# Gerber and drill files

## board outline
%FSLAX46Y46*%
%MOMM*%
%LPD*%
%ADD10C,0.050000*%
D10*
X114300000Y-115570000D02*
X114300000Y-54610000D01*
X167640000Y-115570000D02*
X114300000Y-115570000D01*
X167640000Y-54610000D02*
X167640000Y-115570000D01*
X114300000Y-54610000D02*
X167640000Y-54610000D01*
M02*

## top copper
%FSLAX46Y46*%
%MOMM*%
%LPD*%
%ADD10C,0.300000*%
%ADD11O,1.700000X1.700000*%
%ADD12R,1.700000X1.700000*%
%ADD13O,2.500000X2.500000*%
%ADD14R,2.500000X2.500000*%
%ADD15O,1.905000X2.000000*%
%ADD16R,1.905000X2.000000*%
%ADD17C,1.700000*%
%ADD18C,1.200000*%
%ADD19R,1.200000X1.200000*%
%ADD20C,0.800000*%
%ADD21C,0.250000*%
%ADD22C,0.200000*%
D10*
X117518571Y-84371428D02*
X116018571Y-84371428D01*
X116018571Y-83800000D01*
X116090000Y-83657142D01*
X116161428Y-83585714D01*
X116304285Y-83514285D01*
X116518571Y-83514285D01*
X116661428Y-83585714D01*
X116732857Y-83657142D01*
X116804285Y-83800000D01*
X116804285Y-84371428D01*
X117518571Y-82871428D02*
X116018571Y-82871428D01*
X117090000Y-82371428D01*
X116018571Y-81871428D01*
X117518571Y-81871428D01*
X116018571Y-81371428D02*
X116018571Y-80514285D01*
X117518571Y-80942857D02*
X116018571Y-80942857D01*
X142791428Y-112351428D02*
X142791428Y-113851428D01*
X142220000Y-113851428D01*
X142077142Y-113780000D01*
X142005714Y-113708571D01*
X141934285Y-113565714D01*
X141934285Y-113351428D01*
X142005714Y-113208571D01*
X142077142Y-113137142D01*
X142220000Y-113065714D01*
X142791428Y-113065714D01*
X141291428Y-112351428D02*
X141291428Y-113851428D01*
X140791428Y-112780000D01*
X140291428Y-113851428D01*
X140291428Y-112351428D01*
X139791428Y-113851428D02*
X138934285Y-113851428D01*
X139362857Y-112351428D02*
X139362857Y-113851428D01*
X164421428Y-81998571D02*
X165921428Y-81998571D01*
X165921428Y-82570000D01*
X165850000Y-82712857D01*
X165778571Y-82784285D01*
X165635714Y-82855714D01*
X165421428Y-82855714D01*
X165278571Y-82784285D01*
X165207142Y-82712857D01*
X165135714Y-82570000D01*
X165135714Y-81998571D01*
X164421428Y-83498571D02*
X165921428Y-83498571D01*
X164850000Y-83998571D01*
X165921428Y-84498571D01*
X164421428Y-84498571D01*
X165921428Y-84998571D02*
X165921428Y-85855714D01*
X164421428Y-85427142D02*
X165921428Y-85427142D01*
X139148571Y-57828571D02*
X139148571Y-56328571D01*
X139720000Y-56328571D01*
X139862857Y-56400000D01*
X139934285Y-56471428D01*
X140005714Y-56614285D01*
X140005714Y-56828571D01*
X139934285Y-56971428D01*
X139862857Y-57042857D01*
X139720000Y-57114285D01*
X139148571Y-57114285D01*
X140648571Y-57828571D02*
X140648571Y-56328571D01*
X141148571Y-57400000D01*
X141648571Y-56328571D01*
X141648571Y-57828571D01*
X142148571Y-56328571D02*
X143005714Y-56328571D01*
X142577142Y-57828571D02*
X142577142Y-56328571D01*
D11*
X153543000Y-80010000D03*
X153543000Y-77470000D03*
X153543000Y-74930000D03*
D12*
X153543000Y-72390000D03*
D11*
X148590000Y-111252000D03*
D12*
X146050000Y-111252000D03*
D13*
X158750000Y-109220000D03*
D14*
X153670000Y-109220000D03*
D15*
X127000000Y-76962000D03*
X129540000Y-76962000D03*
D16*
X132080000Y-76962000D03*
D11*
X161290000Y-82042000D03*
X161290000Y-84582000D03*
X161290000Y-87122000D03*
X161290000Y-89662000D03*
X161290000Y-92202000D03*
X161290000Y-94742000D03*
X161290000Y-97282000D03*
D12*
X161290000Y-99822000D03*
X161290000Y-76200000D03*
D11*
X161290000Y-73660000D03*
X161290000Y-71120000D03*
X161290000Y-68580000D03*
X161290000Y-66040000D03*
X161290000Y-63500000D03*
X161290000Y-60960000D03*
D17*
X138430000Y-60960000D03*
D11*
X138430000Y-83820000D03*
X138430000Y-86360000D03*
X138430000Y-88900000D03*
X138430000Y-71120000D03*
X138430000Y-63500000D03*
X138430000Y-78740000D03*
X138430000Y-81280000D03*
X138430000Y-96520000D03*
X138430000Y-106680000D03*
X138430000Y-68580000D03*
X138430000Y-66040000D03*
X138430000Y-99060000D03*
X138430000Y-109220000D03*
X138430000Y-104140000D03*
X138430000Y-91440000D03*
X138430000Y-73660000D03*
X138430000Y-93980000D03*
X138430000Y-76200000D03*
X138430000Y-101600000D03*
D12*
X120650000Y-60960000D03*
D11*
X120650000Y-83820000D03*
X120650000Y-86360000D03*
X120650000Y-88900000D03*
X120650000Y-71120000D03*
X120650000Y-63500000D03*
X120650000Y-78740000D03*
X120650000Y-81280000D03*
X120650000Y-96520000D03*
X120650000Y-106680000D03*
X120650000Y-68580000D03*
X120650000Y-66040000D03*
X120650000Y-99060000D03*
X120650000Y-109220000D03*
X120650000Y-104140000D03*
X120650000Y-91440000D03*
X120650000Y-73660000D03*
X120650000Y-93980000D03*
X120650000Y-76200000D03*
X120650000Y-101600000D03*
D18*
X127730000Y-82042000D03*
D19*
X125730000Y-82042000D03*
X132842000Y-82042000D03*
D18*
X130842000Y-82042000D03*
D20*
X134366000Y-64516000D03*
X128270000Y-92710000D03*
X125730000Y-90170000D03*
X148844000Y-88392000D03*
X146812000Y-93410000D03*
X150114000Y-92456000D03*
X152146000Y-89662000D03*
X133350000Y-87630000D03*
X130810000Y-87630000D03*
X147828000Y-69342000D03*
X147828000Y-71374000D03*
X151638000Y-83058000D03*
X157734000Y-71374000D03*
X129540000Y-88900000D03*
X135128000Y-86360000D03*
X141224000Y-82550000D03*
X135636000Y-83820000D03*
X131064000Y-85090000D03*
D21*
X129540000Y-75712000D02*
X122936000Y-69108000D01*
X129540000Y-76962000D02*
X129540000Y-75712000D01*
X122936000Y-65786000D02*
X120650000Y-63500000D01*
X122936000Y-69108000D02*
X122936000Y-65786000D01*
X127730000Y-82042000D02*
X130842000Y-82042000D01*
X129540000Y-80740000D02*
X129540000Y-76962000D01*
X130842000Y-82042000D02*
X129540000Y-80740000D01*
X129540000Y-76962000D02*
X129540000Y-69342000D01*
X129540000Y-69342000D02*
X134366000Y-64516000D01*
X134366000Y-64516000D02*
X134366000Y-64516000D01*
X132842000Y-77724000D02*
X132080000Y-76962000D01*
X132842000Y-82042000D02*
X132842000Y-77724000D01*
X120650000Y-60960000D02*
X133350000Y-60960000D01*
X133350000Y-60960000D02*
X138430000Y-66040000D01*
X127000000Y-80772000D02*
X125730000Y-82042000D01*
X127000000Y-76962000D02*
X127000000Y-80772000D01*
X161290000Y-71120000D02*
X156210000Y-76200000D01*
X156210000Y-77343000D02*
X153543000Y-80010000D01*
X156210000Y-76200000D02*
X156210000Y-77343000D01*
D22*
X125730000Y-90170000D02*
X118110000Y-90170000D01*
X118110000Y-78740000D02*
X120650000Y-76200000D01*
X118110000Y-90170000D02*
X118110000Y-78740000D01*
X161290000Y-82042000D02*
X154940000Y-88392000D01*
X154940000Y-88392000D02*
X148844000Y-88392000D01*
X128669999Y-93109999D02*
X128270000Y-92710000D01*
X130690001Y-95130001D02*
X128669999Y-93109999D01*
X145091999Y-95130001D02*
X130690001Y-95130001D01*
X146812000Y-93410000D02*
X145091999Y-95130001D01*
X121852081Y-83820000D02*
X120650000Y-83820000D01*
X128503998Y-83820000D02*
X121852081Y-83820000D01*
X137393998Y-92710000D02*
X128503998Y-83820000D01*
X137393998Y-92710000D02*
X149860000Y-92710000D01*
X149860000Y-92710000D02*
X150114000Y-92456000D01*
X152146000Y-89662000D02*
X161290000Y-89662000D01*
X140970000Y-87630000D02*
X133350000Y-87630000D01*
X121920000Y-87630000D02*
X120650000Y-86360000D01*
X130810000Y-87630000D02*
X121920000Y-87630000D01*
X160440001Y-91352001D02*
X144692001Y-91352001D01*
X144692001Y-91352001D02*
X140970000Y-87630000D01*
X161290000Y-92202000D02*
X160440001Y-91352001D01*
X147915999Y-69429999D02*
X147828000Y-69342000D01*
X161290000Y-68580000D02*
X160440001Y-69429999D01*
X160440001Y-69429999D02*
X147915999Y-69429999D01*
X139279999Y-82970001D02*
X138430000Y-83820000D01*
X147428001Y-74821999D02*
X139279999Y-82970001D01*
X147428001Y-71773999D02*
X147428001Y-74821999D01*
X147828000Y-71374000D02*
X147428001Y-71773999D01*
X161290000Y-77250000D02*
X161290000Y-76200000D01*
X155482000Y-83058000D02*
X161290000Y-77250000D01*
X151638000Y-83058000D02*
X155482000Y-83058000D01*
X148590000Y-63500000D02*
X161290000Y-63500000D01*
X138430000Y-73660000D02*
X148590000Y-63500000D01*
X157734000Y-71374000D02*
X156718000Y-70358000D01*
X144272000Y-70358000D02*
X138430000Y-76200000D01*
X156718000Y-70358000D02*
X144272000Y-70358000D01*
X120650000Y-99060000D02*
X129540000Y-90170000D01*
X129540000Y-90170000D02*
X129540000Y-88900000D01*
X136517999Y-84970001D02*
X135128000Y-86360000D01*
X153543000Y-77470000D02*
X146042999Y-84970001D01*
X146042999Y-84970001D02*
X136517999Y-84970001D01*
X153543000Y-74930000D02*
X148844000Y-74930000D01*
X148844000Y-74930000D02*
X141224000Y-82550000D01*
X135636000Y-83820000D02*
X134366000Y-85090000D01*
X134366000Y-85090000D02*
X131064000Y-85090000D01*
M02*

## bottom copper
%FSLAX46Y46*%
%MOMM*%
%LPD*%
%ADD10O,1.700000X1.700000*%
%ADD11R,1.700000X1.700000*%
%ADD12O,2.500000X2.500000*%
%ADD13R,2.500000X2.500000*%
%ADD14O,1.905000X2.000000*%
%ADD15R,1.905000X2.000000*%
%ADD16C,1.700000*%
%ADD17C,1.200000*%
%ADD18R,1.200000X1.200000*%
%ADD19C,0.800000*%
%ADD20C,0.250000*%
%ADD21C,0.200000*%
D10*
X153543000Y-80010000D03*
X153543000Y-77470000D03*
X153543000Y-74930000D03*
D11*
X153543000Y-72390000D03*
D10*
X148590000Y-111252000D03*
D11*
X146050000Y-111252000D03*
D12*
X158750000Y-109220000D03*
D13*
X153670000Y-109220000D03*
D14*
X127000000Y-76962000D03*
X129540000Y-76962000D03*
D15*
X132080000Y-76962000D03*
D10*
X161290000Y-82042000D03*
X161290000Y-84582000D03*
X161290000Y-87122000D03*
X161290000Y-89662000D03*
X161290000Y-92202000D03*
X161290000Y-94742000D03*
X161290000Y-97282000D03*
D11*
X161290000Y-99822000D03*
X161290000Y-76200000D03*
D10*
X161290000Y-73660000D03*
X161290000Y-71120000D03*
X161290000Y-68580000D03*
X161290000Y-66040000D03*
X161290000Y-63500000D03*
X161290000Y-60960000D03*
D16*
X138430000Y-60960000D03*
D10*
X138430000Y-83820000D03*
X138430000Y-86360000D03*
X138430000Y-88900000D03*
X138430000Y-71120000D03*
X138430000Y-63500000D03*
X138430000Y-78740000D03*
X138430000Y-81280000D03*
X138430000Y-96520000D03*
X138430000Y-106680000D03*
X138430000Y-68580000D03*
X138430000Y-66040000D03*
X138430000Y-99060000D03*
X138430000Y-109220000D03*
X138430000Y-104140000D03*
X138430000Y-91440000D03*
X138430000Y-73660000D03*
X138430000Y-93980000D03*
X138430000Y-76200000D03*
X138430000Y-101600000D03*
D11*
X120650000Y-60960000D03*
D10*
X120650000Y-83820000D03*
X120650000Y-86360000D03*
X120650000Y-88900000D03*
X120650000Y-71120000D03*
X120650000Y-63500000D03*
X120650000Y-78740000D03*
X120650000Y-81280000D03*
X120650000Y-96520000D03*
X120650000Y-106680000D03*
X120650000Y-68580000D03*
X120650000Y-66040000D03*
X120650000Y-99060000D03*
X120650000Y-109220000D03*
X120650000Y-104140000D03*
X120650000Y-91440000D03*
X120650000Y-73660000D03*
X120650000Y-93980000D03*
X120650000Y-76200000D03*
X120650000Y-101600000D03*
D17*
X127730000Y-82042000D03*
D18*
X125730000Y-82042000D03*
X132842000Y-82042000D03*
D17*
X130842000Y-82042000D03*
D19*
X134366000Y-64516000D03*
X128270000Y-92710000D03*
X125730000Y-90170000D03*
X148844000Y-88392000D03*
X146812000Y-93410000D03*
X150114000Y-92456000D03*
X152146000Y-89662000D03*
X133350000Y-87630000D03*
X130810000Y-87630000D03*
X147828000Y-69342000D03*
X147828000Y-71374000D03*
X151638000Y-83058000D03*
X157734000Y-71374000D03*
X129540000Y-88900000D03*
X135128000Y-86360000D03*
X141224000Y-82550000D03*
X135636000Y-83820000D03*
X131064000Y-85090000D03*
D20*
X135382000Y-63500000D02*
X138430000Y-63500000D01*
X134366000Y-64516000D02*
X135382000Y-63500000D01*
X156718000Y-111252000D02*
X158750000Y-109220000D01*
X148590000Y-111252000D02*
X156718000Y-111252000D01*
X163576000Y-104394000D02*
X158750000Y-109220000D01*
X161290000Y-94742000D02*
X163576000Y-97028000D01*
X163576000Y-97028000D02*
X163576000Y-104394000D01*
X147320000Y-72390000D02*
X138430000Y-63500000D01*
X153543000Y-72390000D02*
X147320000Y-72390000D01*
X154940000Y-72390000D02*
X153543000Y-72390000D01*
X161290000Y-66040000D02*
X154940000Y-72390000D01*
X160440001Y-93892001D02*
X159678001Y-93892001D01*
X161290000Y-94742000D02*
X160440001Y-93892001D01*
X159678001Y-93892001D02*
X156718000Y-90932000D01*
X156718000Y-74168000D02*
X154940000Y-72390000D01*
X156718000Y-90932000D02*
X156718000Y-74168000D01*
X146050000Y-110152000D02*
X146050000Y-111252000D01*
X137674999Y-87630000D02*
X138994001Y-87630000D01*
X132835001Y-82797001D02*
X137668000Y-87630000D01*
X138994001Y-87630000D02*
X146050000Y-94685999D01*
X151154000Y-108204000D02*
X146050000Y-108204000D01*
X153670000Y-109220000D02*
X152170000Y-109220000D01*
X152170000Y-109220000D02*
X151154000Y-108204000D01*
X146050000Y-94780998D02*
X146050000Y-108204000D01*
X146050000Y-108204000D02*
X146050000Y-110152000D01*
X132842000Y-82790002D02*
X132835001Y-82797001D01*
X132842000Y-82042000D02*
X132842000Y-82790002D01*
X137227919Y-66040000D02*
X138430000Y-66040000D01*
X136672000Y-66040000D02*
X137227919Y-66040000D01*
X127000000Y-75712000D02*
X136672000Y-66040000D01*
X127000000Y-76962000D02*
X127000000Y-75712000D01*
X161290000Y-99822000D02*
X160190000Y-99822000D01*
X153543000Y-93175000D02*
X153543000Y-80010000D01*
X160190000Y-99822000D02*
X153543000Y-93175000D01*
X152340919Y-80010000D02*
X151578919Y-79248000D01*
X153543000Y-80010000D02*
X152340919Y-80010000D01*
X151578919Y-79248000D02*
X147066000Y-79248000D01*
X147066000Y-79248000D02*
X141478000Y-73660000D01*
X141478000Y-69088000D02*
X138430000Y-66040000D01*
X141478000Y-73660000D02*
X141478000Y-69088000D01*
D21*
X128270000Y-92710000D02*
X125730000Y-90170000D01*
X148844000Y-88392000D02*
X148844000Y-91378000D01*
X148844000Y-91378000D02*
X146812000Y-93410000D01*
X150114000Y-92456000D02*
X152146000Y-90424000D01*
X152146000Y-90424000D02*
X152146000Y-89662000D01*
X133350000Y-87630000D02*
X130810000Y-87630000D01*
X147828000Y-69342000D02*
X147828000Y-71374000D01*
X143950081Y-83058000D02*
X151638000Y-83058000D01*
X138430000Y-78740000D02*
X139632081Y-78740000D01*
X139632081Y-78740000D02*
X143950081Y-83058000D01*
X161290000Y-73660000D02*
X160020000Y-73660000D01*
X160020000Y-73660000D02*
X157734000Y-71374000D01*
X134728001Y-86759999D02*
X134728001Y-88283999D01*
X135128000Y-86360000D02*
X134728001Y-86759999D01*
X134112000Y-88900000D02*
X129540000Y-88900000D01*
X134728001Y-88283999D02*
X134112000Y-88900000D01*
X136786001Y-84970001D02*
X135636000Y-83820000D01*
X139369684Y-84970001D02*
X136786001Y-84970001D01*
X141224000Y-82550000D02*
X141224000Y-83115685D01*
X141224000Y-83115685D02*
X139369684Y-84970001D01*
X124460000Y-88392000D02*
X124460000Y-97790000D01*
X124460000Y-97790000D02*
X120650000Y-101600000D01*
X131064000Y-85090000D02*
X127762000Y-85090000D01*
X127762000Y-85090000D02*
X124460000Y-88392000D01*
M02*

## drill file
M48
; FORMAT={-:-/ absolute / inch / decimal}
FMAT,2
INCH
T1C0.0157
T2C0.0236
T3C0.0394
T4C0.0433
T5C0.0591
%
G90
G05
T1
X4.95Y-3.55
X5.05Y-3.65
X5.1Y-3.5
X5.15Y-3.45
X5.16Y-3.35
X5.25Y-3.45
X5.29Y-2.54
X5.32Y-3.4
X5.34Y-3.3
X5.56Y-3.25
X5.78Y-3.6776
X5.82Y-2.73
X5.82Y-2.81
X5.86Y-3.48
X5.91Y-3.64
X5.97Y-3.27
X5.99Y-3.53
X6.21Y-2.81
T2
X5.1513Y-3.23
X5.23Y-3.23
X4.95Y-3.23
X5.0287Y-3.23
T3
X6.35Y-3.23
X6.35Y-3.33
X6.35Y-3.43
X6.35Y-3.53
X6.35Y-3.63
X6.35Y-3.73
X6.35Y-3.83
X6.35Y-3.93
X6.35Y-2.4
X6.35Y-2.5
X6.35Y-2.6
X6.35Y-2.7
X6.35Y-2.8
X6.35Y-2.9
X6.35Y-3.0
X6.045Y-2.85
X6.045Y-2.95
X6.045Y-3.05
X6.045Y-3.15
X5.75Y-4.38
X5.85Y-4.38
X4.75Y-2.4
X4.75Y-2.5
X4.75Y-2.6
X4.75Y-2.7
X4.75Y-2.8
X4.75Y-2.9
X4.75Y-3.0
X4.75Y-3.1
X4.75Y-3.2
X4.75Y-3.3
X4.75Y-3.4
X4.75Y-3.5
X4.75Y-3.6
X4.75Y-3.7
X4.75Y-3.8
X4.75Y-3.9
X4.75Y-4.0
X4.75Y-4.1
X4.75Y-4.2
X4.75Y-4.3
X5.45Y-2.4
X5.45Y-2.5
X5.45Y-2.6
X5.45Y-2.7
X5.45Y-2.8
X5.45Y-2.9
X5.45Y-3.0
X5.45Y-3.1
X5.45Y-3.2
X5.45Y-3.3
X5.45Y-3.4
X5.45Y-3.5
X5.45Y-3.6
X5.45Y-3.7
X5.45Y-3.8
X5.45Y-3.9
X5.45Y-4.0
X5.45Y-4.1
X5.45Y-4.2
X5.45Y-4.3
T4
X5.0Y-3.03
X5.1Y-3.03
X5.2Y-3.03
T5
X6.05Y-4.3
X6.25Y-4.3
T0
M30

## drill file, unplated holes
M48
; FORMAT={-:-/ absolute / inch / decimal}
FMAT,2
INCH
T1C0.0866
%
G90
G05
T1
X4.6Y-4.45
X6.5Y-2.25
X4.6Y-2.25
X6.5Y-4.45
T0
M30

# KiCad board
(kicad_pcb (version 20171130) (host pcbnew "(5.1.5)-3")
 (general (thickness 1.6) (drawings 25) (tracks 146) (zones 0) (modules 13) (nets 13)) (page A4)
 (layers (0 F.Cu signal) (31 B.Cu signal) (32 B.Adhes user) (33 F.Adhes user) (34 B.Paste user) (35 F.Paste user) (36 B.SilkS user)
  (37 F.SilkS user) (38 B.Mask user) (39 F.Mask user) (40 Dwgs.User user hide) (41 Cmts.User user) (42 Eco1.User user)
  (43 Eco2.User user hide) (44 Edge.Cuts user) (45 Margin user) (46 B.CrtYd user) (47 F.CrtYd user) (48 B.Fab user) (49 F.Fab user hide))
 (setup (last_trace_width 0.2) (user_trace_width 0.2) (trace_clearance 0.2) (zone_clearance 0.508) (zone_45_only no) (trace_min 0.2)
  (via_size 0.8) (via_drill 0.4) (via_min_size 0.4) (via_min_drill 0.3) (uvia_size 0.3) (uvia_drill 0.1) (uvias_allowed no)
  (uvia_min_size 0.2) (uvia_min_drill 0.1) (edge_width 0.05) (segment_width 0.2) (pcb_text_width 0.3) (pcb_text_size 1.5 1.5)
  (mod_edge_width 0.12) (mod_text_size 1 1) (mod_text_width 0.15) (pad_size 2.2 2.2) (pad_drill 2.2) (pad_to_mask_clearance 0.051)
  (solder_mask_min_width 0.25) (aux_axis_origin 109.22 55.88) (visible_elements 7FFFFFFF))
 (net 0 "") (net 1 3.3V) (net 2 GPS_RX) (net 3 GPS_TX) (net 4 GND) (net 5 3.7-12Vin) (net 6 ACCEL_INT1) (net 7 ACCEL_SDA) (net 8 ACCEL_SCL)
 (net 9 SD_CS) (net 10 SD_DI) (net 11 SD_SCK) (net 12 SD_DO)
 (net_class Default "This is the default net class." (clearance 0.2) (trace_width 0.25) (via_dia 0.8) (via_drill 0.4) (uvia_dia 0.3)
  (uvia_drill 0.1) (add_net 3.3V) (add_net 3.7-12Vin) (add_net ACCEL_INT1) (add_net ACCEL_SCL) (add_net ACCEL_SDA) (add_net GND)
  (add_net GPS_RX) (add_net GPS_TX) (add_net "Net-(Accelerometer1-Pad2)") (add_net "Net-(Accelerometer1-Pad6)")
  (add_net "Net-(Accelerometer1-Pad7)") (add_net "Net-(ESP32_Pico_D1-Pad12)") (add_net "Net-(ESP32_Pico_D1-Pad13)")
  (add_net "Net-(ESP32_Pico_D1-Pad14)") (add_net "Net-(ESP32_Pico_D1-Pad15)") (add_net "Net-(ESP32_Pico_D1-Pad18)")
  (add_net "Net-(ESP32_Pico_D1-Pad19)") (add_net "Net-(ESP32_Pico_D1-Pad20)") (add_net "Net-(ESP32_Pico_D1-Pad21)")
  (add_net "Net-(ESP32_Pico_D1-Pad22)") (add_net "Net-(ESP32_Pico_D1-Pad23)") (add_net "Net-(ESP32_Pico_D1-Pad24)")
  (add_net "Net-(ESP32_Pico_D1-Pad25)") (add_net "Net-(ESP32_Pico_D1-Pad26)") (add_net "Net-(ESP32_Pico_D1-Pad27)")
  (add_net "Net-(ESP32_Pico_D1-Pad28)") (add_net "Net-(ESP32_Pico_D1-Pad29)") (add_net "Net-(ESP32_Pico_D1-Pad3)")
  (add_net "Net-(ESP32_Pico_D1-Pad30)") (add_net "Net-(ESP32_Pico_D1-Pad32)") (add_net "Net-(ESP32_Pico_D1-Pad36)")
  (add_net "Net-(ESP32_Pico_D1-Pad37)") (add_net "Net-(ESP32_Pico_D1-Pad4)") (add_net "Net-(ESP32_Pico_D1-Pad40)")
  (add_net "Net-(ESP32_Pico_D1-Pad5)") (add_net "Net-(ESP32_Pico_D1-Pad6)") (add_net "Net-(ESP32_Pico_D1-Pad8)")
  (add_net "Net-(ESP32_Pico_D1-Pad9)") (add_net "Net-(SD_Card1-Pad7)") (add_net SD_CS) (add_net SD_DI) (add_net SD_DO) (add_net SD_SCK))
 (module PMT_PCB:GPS (layer B.Cu) (at 139.192 76.2 180)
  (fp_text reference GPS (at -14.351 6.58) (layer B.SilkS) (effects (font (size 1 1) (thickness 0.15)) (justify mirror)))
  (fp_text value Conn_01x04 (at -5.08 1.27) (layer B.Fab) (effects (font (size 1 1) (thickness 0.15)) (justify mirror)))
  (pad 4 thru_hole oval (at -14.351 -3.81 180) (size 1.7 1.7) (drill 1) (layers *.Cu *.Mask) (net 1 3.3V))
  (pad 3 thru_hole oval (at -14.351 -1.27 180) (size 1.7 1.7) (drill 1) (layers *.Cu *.Mask) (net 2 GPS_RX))
  (pad 2 thru_hole oval (at -14.351 1.27 180) (size 1.7 1.7) (drill 1) (layers *.Cu *.Mask) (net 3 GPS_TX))
  (pad 1 thru_hole rect (at -14.351 3.81 180) (size 1.7 1.7) (drill 1) (layers *.Cu *.Mask) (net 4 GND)))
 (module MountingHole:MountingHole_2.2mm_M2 (layer F.Cu) (at 165.1 113.03)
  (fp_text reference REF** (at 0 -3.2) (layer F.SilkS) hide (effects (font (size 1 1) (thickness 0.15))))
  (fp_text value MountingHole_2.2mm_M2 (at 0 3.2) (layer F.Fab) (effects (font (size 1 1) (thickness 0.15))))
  (pad "" np_thru_hole circle (at 0 0) (size 2.2 2.2) (drill 2.2) (layers *.Cu *.Mask)))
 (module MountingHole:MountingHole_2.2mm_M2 (layer F.Cu) (at 116.84 113.03)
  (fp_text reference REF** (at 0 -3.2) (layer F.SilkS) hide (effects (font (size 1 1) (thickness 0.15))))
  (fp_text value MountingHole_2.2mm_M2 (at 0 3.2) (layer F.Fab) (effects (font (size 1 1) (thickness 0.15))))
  (pad "" np_thru_hole circle (at 0 0) (size 2.2 2.2) (drill 2.2) (layers *.Cu *.Mask)))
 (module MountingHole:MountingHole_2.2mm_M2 (layer F.Cu) (at 116.84 57.15)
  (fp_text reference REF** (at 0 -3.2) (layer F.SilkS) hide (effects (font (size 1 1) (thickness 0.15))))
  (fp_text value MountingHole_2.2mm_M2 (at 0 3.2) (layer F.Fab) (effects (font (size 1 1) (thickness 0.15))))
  (pad "" np_thru_hole circle (at 0 0) (size 2.2 2.2) (drill 2.2) (layers *.Cu *.Mask)))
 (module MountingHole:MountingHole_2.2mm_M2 (layer F.Cu) (at 165.1 57.15)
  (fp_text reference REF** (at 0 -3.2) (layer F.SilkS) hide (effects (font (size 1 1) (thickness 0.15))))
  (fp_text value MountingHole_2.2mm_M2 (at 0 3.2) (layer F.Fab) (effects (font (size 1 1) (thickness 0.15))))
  (pad "" np_thru_hole circle (at 0 0) (size 2.2 2.2) (drill 2.2) (layers *.Cu *.Mask)))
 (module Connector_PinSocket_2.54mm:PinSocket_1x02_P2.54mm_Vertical (layer F.Cu) (at 146.05 111.252 90)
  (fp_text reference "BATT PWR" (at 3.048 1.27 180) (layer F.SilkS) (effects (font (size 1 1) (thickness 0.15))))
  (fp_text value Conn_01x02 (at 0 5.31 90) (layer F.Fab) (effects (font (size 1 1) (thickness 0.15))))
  (pad 2 thru_hole oval (at 0 2.54 90) (size 1.7 1.7) (drill 1) (layers *.Cu *.Mask) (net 4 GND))
  (pad 1 thru_hole rect (at 0 0 90) (size 1.7 1.7) (drill 1) (layers *.Cu *.Mask) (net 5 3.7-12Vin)))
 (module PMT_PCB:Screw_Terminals (layer F.Cu) (at 153.67 109.22 90)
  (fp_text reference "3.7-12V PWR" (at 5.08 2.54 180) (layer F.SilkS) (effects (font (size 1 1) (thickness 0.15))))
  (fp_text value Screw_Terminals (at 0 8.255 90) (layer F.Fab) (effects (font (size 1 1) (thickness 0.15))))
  (pad 2 thru_hole oval (at 0 5.08 90) (size 2.5 2.5) (drill 1.5) (layers *.Cu *.Mask) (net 4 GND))
  (pad 1 thru_hole rect (at 0 0 90) (size 2.5 2.5) (drill 1.5) (layers *.Cu *.Mask) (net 5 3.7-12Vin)))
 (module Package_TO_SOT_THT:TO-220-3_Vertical (layer B.Cu) (at 132.08 76.962 180)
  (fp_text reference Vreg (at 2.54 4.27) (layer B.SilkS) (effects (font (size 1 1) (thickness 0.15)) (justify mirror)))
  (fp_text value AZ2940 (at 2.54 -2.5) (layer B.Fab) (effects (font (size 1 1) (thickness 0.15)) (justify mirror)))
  (pad 3 thru_hole oval (at 5.08 0 180) (size 1.905 2) (drill 1.1) (layers *.Cu *.Mask) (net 1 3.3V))
  (pad 2 thru_hole oval (at 2.54 0 180) (size 1.905 2) (drill 1.1) (layers *.Cu *.Mask) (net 4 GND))
  (pad 1 thru_hole rect (at 0 0 180) (size 1.905 2) (drill 1.1) (layers *.Cu *.Mask) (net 5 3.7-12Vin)))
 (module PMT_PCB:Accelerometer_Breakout (layer F.Cu) (at 161.29 99.822 180)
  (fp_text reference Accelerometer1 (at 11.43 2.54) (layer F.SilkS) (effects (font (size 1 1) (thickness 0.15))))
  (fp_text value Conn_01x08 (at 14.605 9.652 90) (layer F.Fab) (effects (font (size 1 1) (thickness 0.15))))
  (pad 8 thru_hole oval (at 0 17.78 180) (size 1.7 1.7) (drill 1) (layers *.Cu *.Mask) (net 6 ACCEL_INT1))
  (pad 7 thru_hole oval (at 0 15.24 180) (size 1.7 1.7) (drill 1) (layers *.Cu *.Mask))
  (pad 6 thru_hole oval (at 0 12.7 180) (size 1.7 1.7) (drill 1) (layers *.Cu *.Mask))
  (pad 5 thru_hole oval (at 0 10.16 180) (size 1.7 1.7) (drill 1) (layers *.Cu *.Mask) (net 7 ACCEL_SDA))
  (pad 4 thru_hole oval (at 0 7.62 180) (size 1.7 1.7) (drill 1) (layers *.Cu *.Mask) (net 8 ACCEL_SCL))
  (pad 3 thru_hole oval (at 0 5.08 180) (size 1.7 1.7) (drill 1) (layers *.Cu *.Mask) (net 4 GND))
  (pad 2 thru_hole oval (at 0 2.54 180) (size 1.7 1.7) (drill 1) (layers *.Cu *.Mask))
  (pad 1 thru_hole rect (at 0 0 180) (size 1.7 1.7) (drill 1) (layers *.Cu *.Mask) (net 1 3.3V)))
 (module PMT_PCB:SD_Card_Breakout (layer F.Cu) (at 161.29 76.2 180)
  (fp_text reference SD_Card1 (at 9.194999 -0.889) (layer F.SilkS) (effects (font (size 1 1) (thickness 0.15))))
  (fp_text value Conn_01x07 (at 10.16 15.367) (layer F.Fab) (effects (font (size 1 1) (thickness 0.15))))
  (pad 1 thru_hole rect (at 0 0 180) (size 1.7 1.7) (drill 1) (layers *.Cu *.Mask) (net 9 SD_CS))
  (pad 2 thru_hole oval (at 0 2.54 180) (size 1.7 1.7) (drill 1) (layers *.Cu *.Mask) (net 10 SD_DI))
  (pad 3 thru_hole oval (at 0 5.08 180) (size 1.7 1.7) (drill 1) (layers *.Cu *.Mask) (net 1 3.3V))
  (pad 4 thru_hole oval (at 0 7.62 180) (size 1.7 1.7) (drill 1) (layers *.Cu *.Mask) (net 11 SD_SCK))
  (pad 5 thru_hole oval (at 0 10.16 180) (size 1.7 1.7) (drill 1) (layers *.Cu *.Mask) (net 4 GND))
  (pad 6 thru_hole oval (at 0 12.7 180) (size 1.7 1.7) (drill 1) (layers *.Cu *.Mask) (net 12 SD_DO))
  (pad 7 thru_hole oval (at 0 15.24 180) (size 1.7 1.7) (drill 1) (layers *.Cu *.Mask)))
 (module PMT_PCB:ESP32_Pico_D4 (layer F.Cu) (at 129.54 59.69)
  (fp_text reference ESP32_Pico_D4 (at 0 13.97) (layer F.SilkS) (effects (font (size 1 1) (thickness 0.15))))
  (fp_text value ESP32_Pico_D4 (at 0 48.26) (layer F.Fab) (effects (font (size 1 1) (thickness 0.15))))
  (pad 40 thru_hole circle (at 8.89 1.27) (size 1.7 1.7) (drill 1) (layers *.Cu *.Mask))
  (pad 31 thru_hole oval (at 8.89 24.13) (size 1.7 1.7) (drill 1) (layers *.Cu *.Mask) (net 11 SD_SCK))
  (pad 30 thru_hole oval (at 8.89 26.67) (size 1.7 1.7) (drill 1) (layers *.Cu *.Mask))
  (pad 29 thru_hole oval (at 8.89 29.21) (size 1.7 1.7) (drill 1) (layers *.Cu *.Mask))
  (pad 36 thru_hole oval (at 8.89 11.43) (size 1.7 1.7) (drill 1) (layers *.Cu *.Mask))
  (pad 39 thru_hole oval (at 8.89 3.81) (size 1.7 1.7) (drill 1) (layers *.Cu *.Mask) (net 4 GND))
  (pad 33 thru_hole oval (at 8.89 19.05) (size 1.7 1.7) (drill 1) (layers *.Cu *.Mask) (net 9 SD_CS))
  (pad 32 thru_hole oval (at 8.89 21.59) (size 1.7 1.7) (drill 1) (layers *.Cu *.Mask))
  (pad 26 thru_hole oval (at 8.89 36.83) (size 1.7 1.7) (drill 1) (layers *.Cu *.Mask))
  (pad 22 thru_hole oval (at 8.89 46.99) (size 1.7 1.7) (drill 1) (layers *.Cu *.Mask))
  (pad 37 thru_hole oval (at 8.89 8.89) (size 1.7 1.7) (drill 1) (layers *.Cu *.Mask))
  (pad 38 thru_hole oval (at 8.89 6.35) (size 1.7 1.7) (drill 1) (layers *.Cu *.Mask) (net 1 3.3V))
  (pad 25 thru_hole oval (at 8.89 39.37) (size 1.7 1.7) (drill 1) (layers *.Cu *.Mask))
  (pad 21 thru_hole oval (at 8.89 49.53) (size 1.7 1.7) (drill 1) (layers *.Cu *.Mask))
  (pad 23 thru_hole oval (at 8.89 44.45) (size 1.7 1.7) (drill 1) (layers *.Cu *.Mask))
  (pad 28 thru_hole oval (at 8.89 31.75) (size 1.7 1.7) (drill 1) (layers *.Cu *.Mask))
  (pad 35 thru_hole oval (at 8.89 13.97) (size 1.7 1.7) (drill 1) (layers *.Cu *.Mask) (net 12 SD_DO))
  (pad 27 thru_hole oval (at 8.89 34.29) (size 1.7 1.7) (drill 1) (layers *.Cu *.Mask))
  (pad 34 thru_hole oval (at 8.89 16.51) (size 1.7 1.7) (drill 1) (layers *.Cu *.Mask) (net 10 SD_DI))
  (pad 24 thru_hole oval (at 8.89 41.91) (size 1.7 1.7) (drill 1) (layers *.Cu *.Mask))
  (pad 1 thru_hole rect (at -8.89 1.27) (size 1.7 1.7) (drill 1) (layers *.Cu *.Mask) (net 1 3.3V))
  (pad 10 thru_hole oval (at -8.89 24.13) (size 1.7 1.7) (drill 1) (layers *.Cu *.Mask) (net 7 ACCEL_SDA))
  (pad 11 thru_hole oval (at -8.89 26.67) (size 1.7 1.7) (drill 1) (layers *.Cu *.Mask) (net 8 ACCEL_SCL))
  (pad 12 thru_hole oval (at -8.89 29.21) (size 1.7 1.7) (drill 1) (layers *.Cu *.Mask))
  (pad 5 thru_hole oval (at -8.89 11.43) (size 1.7 1.7) (drill 1) (layers *.Cu *.Mask))
  (pad 2 thru_hole oval (at -8.89 3.81) (size 1.7 1.7) (drill 1) (layers *.Cu *.Mask) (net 4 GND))
  (pad 8 thru_hole oval (at -8.89 19.05) (size 1.7 1.7) (drill 1) (layers *.Cu *.Mask))
  (pad 9 thru_hole oval (at -8.89 21.59) (size 1.7 1.7) (drill 1) (layers *.Cu *.Mask))
  (pad 15 thru_hole oval (at -8.89 36.83) (size 1.7 1.7) (drill 1) (layers *.Cu *.Mask))
  (pad 19 thru_hole oval (at -8.89 46.99) (size 1.7 1.7) (drill 1) (layers *.Cu *.Mask))
  (pad 4 thru_hole oval (at -8.89 8.89) (size 1.7 1.7) (drill 1) (layers *.Cu *.Mask))
  (pad 3 thru_hole oval (at -8.89 6.35) (size 1.7 1.7) (drill 1) (layers *.Cu *.Mask))
  (pad 16 thru_hole oval (at -8.89 39.37) (size 1.7 1.7) (drill 1) (layers *.Cu *.Mask) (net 2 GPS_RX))
  (pad 20 thru_hole oval (at -8.89 49.53) (size 1.7 1.7) (drill 1) (layers *.Cu *.Mask))
  (pad 18 thru_hole oval (at -8.89 44.45) (size 1.7 1.7) (drill 1) (layers *.Cu *.Mask))
  (pad 13 thru_hole oval (at -8.89 31.75) (size 1.7 1.7) (drill 1) (layers *.Cu *.Mask))
  (pad 6 thru_hole oval (at -8.89 13.97) (size 1.7 1.7) (drill 1) (layers *.Cu *.Mask))
  (pad 14 thru_hole oval (at -8.89 34.29) (size 1.7 1.7) (drill 1) (layers *.Cu *.Mask))
  (pad 7 thru_hole oval (at -8.89 16.51) (size 1.7 1.7) (drill 1) (layers *.Cu *.Mask) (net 6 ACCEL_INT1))
  (pad 17 thru_hole oval (at -8.89 41.91) (size 1.7 1.7) (drill 1) (layers *.Cu *.Mask) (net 3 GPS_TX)))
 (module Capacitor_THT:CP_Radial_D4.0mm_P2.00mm (layer B.Cu) (at 125.73 82.042)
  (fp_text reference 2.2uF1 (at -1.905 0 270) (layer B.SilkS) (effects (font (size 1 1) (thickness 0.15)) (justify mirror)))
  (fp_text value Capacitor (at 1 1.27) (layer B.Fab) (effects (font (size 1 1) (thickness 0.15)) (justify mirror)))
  (pad 2 thru_hole circle (at 2 0) (size 1.2 1.2) (drill 0.6) (layers *.Cu *.Mask) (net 4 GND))
  (pad 1 thru_hole rect (at 0 0) (size 1.2 1.2) (drill 0.6) (layers *.Cu *.Mask) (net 1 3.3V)))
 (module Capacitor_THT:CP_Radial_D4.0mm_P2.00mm (layer B.Cu) (at 132.842 82.042 180)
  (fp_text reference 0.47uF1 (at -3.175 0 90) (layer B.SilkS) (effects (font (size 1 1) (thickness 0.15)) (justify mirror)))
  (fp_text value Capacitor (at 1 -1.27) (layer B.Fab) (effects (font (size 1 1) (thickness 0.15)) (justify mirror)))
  (pad 1 thru_hole rect (at 0 0 180) (size 1.2 1.2) (drill 0.6) (layers *.Cu *.Mask) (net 5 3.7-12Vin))
  (pad 2 thru_hole circle (at 2 0 180) (size 1.2 1.2) (drill 0.6) (layers *.Cu *.Mask) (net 4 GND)))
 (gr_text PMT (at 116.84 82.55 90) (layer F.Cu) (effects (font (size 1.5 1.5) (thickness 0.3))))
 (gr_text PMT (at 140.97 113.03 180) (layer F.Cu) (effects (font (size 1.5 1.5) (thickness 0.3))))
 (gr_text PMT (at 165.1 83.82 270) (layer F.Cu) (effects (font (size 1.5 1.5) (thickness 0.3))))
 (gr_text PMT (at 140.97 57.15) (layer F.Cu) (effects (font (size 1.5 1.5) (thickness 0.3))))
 (gr_line (start 114.3 115.57) (end 114.3 54.61) (layer Edge.Cuts) (width 0.05))
 (gr_line (start 167.64 115.57) (end 114.3 115.57) (layer Edge.Cuts) (width 0.05))
 (gr_line (start 167.64 54.61) (end 167.64 115.57) (layer Edge.Cuts) (width 0.05))
 (gr_line (start 114.3 54.61) (end 167.64 54.61) (layer Edge.Cuts) (width 0.05))
 (segment (start 129.54 75.712) (end 122.936 69.108) (width 0.25) (layer F.Cu) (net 4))
 (segment (start 129.54 76.962) (end 129.54 75.712) (width 0.25) (layer F.Cu) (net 4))
 (segment (start 122.936 65.786) (end 120.65 63.5) (width 0.25) (layer F.Cu) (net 4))
 (segment (start 122.936 69.108) (end 122.936 65.786) (width 0.25) (layer F.Cu) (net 4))
 (segment (start 127.73 82.042) (end 130.842 82.042) (width 0.25) (layer F.Cu) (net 4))
 (segment (start 129.54 80.74) (end 129.54 76.962) (width 0.25) (layer F.Cu) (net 4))
 (segment (start 130.842 82.042) (end 129.54 80.74) (width 0.25) (layer F.Cu) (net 4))
 (segment (start 129.54 76.962) (end 129.54 69.342) (width 0.25) (layer F.Cu) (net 4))
 (segment (start 129.54 69.342) (end 134.366 64.516) (width 0.25) (layer F.Cu) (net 4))
 (segment (start 134.366 64.516) (end 134.366 64.516) (width 0.25) (layer F.Cu) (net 4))
 (via (at 134.366 64.516) (size 0.8) (drill 0.4) (layers F.Cu B.Cu) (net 4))
 (segment (start 135.382 63.5) (end 138.43 63.5) (width 0.25) (layer B.Cu) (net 4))
 (segment (start 134.366 64.516) (end 135.382 63.5) (width 0.25) (layer B.Cu) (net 4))
 (segment (start 156.718 111.252) (end 158.75 109.22) (width 0.25) (layer B.Cu) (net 4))
 (segment (start 148.59 111.252) (end 156.718 111.252) (width 0.25) (layer B.Cu) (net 4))
 (segment (start 163.576 104.394) (end 158.75 109.22) (width 0.25) (layer B.Cu) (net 4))
 (segment (start 161.29 94.742) (end 163.576 97.028) (width 0.25) (layer B.Cu) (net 4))
 (segment (start 163.576 97.028) (end 163.576 104.394) (width 0.25) (layer B.Cu) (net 4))
 (segment (start 147.32 72.39) (end 138.43 63.5) (width 0.25) (layer B.Cu) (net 4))
 (segment (start 153.543 72.39) (end 147.32 72.39) (width 0.25) (layer B.Cu) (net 4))
 (segment (start 154.94 72.39) (end 153.543 72.39) (width 0.25) (layer B.Cu) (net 4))
 (segment (start 161.29 66.04) (end 154.94 72.39) (width 0.25) (layer B.Cu) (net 4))
 (segment (start 160.440001 93.892001) (end 159.678001 93.892001) (width 0.25) (layer B.Cu) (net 4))
 (segment (start 161.29 94.742) (end 160.440001 93.892001) (width 0.25) (layer B.Cu) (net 4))
 (segment (start 159.678001 93.892001) (end 156.718 90.932) (width 0.25) (layer B.Cu) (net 4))
 (segment (start 156.718 74.168) (end 154.94 72.39) (width 0.25) (layer B.Cu) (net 4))
 (segment (start 156.718 90.932) (end 156.718 74.168) (width 0.25) (layer B.Cu) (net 4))
 (segment (start 132.842 77.724) (end 132.08 76.962) (width 0.25) (layer F.Cu) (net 5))
 (segment (start 132.842 82.042) (end 132.842 77.724) (width 0.25) (layer F.Cu) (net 5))
 (segment (start 146.05 110.152) (end 146.05 111.252) (width 0.25) (layer B.Cu) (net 5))
 (segment (start 137.674999 87.63) (end 138.994001 87.63) (width 0.25) (layer B.Cu) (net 5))
 (segment (start 132.835001 82.797001) (end 137.668 87.63) (width 0.25) (layer B.Cu) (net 5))
 (segment (start 138.994001 87.63) (end 146.05 94.685999) (width 0.25) (layer B.Cu) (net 5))
 (segment (start 151.154 108.204) (end 146.05 108.204) (width 0.25) (layer B.Cu) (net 5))
 (segment (start 153.67 109.22) (end 152.17 109.22) (width 0.25) (layer B.Cu) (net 5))
 (segment (start 152.17 109.22) (end 151.154 108.204) (width 0.25) (layer B.Cu) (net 5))
 (segment (start 146.05 94.780998) (end 146.05 108.204) (width 0.25) (layer B.Cu) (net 5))
 (segment (start 146.05 108.204) (end 146.05 110.152) (width 0.25) (layer B.Cu) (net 5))
 (segment (start 132.842 82.790002) (end 132.835001 82.797001) (width 0.25) (layer B.Cu) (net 5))
 (segment (start 132.842 82.042) (end 132.842 82.790002) (width 0.25) (layer B.Cu) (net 5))
 (segment (start 120.65 60.96) (end 133.35 60.96) (width 0.25) (layer F.Cu) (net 1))
 (segment (start 133.35 60.96) (end 138.43 66.04) (width 0.25) (layer F.Cu) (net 1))
 (segment (start 127 80.772) (end 125.73 82.042) (width 0.25) (layer F.Cu) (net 1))
 (segment (start 127 76.962) (end 127 80.772) (width 0.25) (layer F.Cu) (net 1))
 (segment (start 137.227919 66.04) (end 138.43 66.04) (width 0.25) (layer B.Cu) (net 1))
 (segment (start 136.672 66.04) (end 137.227919 66.04) (width 0.25) (layer B.Cu) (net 1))
 (segment (start 127 75.712) (end 136.672 66.04) (width 0.25) (layer B.Cu) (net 1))
 (segment (start 127 76.962) (end 127 75.712) (width 0.25) (layer B.Cu) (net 1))
 (segment (start 161.29 99.822) (end 160.19 99.822) (width 0.25) (layer B.Cu) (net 1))
 (segment (start 153.543 93.175) (end 153.543 80.01) (width 0.25) (layer B.Cu) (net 1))
 (segment (start 160.19 99.822) (end 153.543 93.175) (width 0.25) (layer B.Cu) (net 1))
 (segment (start 152.340919 80.01) (end 151.578919 79.248) (width 0.25) (layer B.Cu) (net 1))
 (segment (start 153.543 80.01) (end 152.340919 80.01) (width 0.25) (layer B.Cu) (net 1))
 (segment (start 151.578919 79.248) (end 147.066 79.248) (width 0.25) (layer B.Cu) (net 1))
 (segment (start 147.066 79.248) (end 141.478 73.66) (width 0.25) (layer B.Cu) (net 1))
 (segment (start 141.478 69.088) (end 138.43 66.04) (width 0.25) (layer B.Cu) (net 1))
 (segment (start 141.478 73.66) (end 141.478 69.088) (width 0.25) (layer B.Cu) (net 1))
 (segment (start 161.29 71.12) (end 156.21 76.2) (width 0.25) (layer F.Cu) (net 1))
 (segment (start 156.21 77.343) (end 153.543 80.01) (width 0.25) (layer F.Cu) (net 1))
 (segment (start 156.21 76.2) (end 156.21 77.343) (width 0.25) (layer F.Cu) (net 1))
 (via (at 128.27 92.71) (size 0.8) (drill 0.4) (layers F.Cu B.Cu) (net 6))
 (segment (start 128.27 92.71) (end 125.73 90.17) (width 0.2) (layer B.Cu) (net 6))
 (via (at 125.73 90.17) (size 0.8) (drill 0.4) (layers F.Cu B.Cu) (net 6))
 (segment (start 125.73 90.17) (end 118.11 90.17) (width 0.2) (layer F.Cu) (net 6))
 (segment (start 118.11 78.74) (end 120.65 76.2) (width 0.2) (layer F.Cu) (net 6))
 (segment (start 118.11 90.17) (end 118.11 78.74) (width 0.2) (layer F.Cu) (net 6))
 (via (at 148.844 88.392) (size 0.8) (drill 0.4) (layers F.Cu B.Cu) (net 6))
 (segment (start 161.29 82.042) (end 154.94 88.392) (width 0.2) (layer F.Cu) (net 6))
 (segment (start 154.94 88.392) (end 148.844 88.392) (width 0.2) (layer F.Cu) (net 6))
 (via (at 146.812 93.41) (size 0.8) (drill 0.4) (layers F.Cu B.Cu) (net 6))
 (segment (start 148.844 88.392) (end 148.844 91.378) (width 0.2) (layer B.Cu) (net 6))
 (segment (start 148.844 91.378) (end 146.812 93.41) (width 0.2) (layer B.Cu) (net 6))
 (segment (start 128.669999 93.109999) (end 128.27 92.71) (width 0.2) (layer F.Cu) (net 6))
 (segment (start 130.690001 95.130001) (end 128.669999 93.109999) (width 0.2) (layer F.Cu) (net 6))
 (segment (start 145.091999 95.130001) (end 130.690001 95.130001) (width 0.2) (layer F.Cu) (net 6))
 (segment (start 146.812 93.41) (end 145.091999 95.130001) (width 0.2) (layer F.Cu) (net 6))
 (segment (start 121.852081 83.82) (end 120.65 83.82) (width 0.2) (layer F.Cu) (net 7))
 (segment (start 128.503998 83.82) (end 121.852081 83.82) (width 0.2) (layer F.Cu) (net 7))
 (segment (start 137.393998 92.71) (end 128.503998 83.82) (width 0.2) (layer F.Cu) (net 7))
 (via (at 150.114 92.456) (size 0.8) (drill 0.4) (layers F.Cu B.Cu) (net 7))
 (segment (start 137.393998 92.71) (end 149.86 92.71) (width 0.2) (layer F.Cu) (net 7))
 (segment (start 149.86 92.71) (end 150.114 92.456) (width 0.2) (layer F.Cu) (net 7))
 (via (at 152.146 89.662) (size 0.8) (drill 0.4) (layers F.Cu B.Cu) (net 7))
 (segment (start 150.114 92.456) (end 152.146 90.424) (width 0.2) (layer B.Cu) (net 7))
 (segment (start 152.146 90.424) (end 152.146 89.662) (width 0.2) (layer B.Cu) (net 7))
 (segment (start 152.146 89.662) (end 161.29 89.662) (width 0.2) (layer F.Cu) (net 7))
 (via (at 133.35 87.63) (size 0.8) (drill 0.4) (layers F.Cu B.Cu) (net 8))
 (segment (start 140.97 87.63) (end 133.35 87.63) (width 0.2) (layer F.Cu) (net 8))
 (via (at 130.81 87.63) (size 0.8) (drill 0.4) (layers F.Cu B.Cu) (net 8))
 (segment (start 133.35 87.63) (end 130.81 87.63) (width 0.2) (layer B.Cu) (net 8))
 (segment (start 121.92 87.63) (end 120.65 86.36) (width 0.2) (layer F.Cu) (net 8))
 (segment (start 130.81 87.63) (end 121.92 87.63) (width 0.2) (layer F.Cu) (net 8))
 (segment (start 160.440001 91.352001) (end 144.692001 91.352001) (width 0.2) (layer F.Cu) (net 8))
 (segment (start 144.692001 91.352001) (end 140.97 87.63) (width 0.2) (layer F.Cu) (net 8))
 (segment (start 161.29 92.202) (end 160.440001 91.352001) (width 0.2) (layer F.Cu) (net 8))
 (segment (start 147.915999 69.429999) (end 147.828 69.342) (width 0.2) (layer F.Cu) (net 11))
 (segment (start 161.29 68.58) (end 160.440001 69.429999) (width 0.2) (layer F.Cu) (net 11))
 (via (at 147.828 69.342) (size 0.8) (drill 0.4) (layers F.Cu B.Cu) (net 11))
 (segment (start 160.440001 69.429999) (end 147.915999 69.429999) (width 0.2) (layer F.Cu) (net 11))
 (via (at 147.828 71.374) (size 0.8) (drill 0.4) (layers F.Cu B.Cu) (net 11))
 (segment (start 147.828 69.342) (end 147.828 71.374) (width 0.2) (layer B.Cu) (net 11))
 (segment (start 139.279999 82.970001) (end 138.43 83.82) (width 0.2) (layer F.Cu) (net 11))
 (segment (start 147.428001 74.821999) (end 139.279999 82.970001) (width 0.2) (layer F.Cu) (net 11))
 (segment (start 147.428001 71.773999) (end 147.428001 74.821999) (width 0.2) (layer F.Cu) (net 11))
 (segment (start 147.828 71.374) (end 147.428001 71.773999) (width 0.2) (layer F.Cu) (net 11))
 (via (at 151.638 83.058) (size 0.8) (drill 0.4) (layers F.Cu B.Cu) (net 9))
 (segment (start 143.950081 83.058) (end 151.638 83.058) (width 0.2) (layer B.Cu) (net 9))
 (segment (start 138.43 78.74) (end 139.632081 78.74) (width 0.2) (layer B.Cu) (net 9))
 (segment (start 139.632081 78.74) (end 143.950081 83.058) (width 0.2) (layer B.Cu) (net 9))
 (segment (start 161.29 77.25) (end 161.29 76.2) (width 0.2) (layer F.Cu) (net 9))
 (segment (start 155.482 83.058) (end 161.29 77.25) (width 0.2) (layer F.Cu) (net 9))
 (segment (start 151.638 83.058) (end 155.482 83.058) (width 0.2) (layer F.Cu) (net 9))
 (segment (start 148.59 63.5) (end 161.29 63.5) (width 0.2) (layer F.Cu) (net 12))
 (segment (start 138.43 73.66) (end 148.59 63.5) (width 0.2) (layer F.Cu) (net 12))
 (via (at 157.734 71.374) (size 0.8) (drill 0.4) (layers F.Cu B.Cu) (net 10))
 (segment (start 161.29 73.66) (end 160.02 73.66) (width 0.2) (layer B.Cu) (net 10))
 (segment (start 160.02 73.66) (end 157.734 71.374) (width 0.2) (layer B.Cu) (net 10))
 (segment (start 157.734 71.374) (end 156.718 70.358) (width 0.2) (layer F.Cu) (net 10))
 (segment (start 144.272 70.358) (end 138.43 76.2) (width 0.2) (layer F.Cu) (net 10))
 (segment (start 156.718 70.358) (end 144.272 70.358) (width 0.2) (layer F.Cu) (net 10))
 (via (at 129.54 88.9) (size 0.8) (drill 0.4) (layers F.Cu B.Cu) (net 2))
 (segment (start 120.65 99.06) (end 129.54 90.17) (width 0.2) (layer F.Cu) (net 2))
 (segment (start 129.54 90.17) (end 129.54 88.9) (width 0.2) (layer F.Cu) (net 2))
 (via (at 135.128 86.36) (size 0.8) (drill 0.4) (layers F.Cu B.Cu) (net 2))
 (segment (start 136.517999 84.970001) (end 135.128 86.36) (width 0.2) (layer F.Cu) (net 2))
 (segment (start 153.543 77.47) (end 146.042999 84.970001) (width 0.2) (layer F.Cu) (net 2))
 (segment (start 146.042999 84.970001) (end 136.517999 84.970001) (width 0.2) (layer F.Cu) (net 2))
 (segment (start 134.728001 86.759999) (end 134.728001 88.283999) (width 0.2) (layer B.Cu) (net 2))
 (segment (start 135.128 86.36) (end 134.728001 86.759999) (width 0.2) (layer B.Cu) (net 2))
 (segment (start 134.112 88.9) (end 129.54 88.9) (width 0.2) (layer B.Cu) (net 2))
 (segment (start 134.728001 88.283999) (end 134.112 88.9) (width 0.2) (layer B.Cu) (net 2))
 (via (at 141.224 82.55) (size 0.8) (drill 0.4) (layers F.Cu B.Cu) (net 3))
 (segment (start 153.543 74.93) (end 148.844 74.93) (width 0.2) (layer F.Cu) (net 3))
 (segment (start 148.844 74.93) (end 141.224 82.55) (width 0.2) (layer F.Cu) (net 3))
 (segment (start 136.786001 84.970001) (end 135.636 83.82) (width 0.2) (layer B.Cu) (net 3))
 (segment (start 139.369684 84.970001) (end 136.786001 84.970001) (width 0.2) (layer B.Cu) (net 3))
 (segment (start 141.224 82.55) (end 141.224 83.115685) (width 0.2) (layer B.Cu) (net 3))
 (via (at 135.636 83.82) (size 0.8) (drill 0.4) (layers F.Cu B.Cu) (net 3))
 (segment (start 141.224 83.115685) (end 139.369684 84.970001) (width 0.2) (layer B.Cu) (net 3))
 (via (at 131.064 85.09) (size 0.8) (drill 0.4) (layers F.Cu B.Cu) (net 3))
 (segment (start 135.636 83.82) (end 134.366 85.09) (width 0.2) (layer F.Cu) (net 3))
 (segment (start 134.366 85.09) (end 131.064 85.09) (width 0.2) (layer F.Cu) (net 3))
 (segment (start 124.46 88.392) (end 124.46 97.79) (width 0.2) (layer B.Cu) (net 3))
 (segment (start 124.46 97.79) (end 120.65 101.6) (width 0.2) (layer B.Cu) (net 3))
 (segment (start 131.064 85.09) (end 127.762 85.09) (width 0.2) (layer B.Cu) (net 3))
 (segment (start 127.762 85.09) (end 124.46 88.392) (width 0.2) (layer B.Cu) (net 3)))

